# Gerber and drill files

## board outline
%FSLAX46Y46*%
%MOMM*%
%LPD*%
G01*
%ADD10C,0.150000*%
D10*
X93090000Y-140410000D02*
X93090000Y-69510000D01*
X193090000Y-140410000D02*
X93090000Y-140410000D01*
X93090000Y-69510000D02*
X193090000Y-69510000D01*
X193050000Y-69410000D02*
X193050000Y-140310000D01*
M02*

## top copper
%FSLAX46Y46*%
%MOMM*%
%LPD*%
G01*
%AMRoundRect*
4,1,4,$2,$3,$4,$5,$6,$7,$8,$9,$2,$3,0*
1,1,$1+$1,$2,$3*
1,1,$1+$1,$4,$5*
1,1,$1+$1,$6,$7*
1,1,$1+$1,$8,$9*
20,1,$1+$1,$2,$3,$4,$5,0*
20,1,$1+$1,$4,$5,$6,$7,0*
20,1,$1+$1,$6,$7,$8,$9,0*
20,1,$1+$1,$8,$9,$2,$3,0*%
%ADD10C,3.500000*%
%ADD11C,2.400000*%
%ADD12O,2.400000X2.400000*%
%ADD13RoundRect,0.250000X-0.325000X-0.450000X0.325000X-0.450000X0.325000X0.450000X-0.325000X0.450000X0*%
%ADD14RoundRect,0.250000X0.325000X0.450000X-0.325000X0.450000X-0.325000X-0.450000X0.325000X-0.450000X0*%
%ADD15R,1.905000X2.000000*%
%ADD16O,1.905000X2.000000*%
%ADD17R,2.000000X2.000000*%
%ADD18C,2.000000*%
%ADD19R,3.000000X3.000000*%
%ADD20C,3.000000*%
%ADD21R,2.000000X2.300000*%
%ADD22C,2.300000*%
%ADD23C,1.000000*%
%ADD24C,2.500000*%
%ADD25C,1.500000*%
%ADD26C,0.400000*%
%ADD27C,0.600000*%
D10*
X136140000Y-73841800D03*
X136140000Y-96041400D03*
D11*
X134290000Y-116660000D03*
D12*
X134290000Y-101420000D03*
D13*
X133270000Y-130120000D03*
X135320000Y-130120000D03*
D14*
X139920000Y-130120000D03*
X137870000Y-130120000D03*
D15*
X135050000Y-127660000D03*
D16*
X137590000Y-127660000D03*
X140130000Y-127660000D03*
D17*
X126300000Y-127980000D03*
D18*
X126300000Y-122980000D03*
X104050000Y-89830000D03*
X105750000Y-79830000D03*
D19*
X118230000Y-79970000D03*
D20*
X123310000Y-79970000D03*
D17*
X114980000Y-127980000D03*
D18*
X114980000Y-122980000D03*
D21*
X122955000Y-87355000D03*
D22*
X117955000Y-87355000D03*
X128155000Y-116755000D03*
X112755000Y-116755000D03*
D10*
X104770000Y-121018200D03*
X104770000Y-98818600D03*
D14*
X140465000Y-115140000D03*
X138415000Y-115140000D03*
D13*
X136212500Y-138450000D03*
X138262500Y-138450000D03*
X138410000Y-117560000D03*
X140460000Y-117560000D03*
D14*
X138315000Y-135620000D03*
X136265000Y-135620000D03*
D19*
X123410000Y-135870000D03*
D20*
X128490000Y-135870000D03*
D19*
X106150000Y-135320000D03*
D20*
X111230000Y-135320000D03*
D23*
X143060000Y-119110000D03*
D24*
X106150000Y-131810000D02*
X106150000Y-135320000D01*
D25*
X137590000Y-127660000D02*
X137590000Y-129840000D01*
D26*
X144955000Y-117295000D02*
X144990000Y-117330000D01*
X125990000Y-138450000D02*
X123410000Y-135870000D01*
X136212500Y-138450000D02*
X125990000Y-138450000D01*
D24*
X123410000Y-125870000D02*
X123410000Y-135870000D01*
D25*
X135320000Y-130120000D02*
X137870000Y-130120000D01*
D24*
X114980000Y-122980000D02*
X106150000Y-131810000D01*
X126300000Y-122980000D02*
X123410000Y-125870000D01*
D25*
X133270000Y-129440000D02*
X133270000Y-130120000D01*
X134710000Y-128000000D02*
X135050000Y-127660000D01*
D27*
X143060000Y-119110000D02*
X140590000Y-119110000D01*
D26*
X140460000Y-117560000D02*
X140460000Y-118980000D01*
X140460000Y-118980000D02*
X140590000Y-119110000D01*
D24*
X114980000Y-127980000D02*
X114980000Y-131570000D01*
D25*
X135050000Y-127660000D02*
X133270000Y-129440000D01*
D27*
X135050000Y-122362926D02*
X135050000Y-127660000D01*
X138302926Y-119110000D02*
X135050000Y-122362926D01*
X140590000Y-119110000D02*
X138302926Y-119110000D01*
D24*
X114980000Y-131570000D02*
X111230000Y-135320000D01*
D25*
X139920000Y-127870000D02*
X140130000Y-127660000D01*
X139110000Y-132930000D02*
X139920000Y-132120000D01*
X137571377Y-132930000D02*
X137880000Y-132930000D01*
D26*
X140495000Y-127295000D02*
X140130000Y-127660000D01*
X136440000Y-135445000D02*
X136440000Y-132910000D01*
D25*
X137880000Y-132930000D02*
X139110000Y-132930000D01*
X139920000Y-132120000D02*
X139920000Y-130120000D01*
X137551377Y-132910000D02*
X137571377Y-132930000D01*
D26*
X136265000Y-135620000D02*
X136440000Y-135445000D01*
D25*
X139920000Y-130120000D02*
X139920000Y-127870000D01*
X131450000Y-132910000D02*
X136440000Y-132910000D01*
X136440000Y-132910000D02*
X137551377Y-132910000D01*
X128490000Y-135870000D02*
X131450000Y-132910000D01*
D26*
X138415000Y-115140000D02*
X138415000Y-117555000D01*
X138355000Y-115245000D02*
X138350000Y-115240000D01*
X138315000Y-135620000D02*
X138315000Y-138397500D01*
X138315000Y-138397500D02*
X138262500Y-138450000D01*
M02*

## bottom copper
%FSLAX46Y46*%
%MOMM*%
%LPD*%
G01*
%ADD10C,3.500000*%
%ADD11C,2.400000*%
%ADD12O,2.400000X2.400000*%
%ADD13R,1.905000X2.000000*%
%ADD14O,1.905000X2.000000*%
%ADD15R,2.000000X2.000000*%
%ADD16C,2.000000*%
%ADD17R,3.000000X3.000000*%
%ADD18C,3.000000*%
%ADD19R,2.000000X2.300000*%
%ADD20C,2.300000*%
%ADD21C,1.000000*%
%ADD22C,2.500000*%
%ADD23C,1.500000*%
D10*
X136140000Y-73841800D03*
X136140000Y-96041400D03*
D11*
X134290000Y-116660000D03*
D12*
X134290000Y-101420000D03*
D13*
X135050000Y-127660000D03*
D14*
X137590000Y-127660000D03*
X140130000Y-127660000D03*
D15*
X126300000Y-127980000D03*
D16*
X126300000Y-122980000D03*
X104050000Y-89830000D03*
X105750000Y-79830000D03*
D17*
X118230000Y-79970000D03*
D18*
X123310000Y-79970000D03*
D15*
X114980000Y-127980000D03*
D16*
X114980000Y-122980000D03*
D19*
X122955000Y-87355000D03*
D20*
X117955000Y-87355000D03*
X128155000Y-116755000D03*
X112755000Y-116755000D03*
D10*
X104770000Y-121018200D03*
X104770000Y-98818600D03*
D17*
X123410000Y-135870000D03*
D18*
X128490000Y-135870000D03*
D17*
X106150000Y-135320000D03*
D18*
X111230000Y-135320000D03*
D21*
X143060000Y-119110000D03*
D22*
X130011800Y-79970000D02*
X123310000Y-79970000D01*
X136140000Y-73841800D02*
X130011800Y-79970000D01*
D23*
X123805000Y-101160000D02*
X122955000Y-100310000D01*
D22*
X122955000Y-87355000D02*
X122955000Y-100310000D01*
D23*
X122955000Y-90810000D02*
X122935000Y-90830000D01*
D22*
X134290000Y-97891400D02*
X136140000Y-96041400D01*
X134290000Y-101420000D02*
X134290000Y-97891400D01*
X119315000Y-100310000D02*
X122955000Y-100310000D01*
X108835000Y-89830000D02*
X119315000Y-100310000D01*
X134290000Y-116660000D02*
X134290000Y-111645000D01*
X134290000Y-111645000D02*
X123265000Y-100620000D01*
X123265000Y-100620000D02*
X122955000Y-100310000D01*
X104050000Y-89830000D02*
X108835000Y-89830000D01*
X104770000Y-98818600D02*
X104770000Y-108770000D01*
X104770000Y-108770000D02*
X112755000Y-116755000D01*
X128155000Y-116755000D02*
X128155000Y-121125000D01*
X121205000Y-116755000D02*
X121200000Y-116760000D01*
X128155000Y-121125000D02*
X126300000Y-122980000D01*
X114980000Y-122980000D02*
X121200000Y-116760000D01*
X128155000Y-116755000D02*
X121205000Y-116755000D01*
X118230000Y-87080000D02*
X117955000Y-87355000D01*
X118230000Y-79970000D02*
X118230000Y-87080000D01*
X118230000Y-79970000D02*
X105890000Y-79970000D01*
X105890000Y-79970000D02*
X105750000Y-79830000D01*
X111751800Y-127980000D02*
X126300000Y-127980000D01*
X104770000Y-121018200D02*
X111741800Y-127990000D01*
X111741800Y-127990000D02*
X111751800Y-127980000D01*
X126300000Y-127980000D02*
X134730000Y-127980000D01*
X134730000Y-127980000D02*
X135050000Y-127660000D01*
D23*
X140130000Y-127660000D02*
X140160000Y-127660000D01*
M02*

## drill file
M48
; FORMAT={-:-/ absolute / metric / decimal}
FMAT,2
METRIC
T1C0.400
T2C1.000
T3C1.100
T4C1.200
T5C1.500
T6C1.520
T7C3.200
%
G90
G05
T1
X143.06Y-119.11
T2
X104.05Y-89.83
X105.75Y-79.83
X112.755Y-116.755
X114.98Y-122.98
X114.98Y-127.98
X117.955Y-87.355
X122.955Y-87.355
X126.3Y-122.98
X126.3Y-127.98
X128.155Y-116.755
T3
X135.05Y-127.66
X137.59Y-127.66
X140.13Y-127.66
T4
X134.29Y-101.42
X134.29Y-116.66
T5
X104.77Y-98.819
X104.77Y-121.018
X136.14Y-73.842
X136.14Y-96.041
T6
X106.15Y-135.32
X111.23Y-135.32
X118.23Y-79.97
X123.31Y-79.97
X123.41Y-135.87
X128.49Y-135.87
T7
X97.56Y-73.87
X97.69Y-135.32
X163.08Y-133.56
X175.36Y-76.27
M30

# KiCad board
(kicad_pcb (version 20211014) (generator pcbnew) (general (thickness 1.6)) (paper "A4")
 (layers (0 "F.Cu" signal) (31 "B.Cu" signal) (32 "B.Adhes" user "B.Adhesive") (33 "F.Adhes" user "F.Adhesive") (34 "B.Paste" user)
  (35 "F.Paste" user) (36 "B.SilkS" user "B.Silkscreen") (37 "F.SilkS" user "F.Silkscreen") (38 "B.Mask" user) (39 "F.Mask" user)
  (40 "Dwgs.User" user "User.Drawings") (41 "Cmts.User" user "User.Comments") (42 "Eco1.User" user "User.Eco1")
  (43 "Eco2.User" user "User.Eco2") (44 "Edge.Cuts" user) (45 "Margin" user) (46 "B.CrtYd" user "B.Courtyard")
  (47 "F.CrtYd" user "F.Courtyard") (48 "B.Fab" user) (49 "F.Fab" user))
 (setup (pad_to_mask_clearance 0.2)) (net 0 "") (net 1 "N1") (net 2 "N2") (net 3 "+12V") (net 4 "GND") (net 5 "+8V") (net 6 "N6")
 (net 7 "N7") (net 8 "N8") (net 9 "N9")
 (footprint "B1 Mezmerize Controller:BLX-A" (layer "F.Cu") (at 136.14 84.84 -90)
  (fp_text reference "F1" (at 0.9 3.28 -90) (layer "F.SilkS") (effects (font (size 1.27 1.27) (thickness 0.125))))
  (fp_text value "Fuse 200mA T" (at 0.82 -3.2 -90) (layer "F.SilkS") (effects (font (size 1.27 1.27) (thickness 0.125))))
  (pad "1" thru_hole circle locked (at -10.9982 0 270) (size 3.5 3.5) (drill 1.5) (layers *.Cu *.Mask "F.SilkS") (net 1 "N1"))
  (pad "2" thru_hole circle locked (at 11.2014 0 270) (size 3.5 3.5) (drill 1.5) (layers *.Cu *.Mask "F.SilkS") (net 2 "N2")))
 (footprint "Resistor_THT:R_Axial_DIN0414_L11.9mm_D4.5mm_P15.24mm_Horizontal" (layer "F.Cu") (at 134.29 116.66 90)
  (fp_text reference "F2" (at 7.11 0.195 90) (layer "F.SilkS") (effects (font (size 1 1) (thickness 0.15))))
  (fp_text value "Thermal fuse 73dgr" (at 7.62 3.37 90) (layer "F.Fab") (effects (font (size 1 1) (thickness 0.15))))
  (pad "1" thru_hole circle (at 0 0 90) (size 2.4 2.4) (drill 1.2) (layers *.Cu *.Mask) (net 2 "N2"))
  (pad "2" thru_hole oval (at 15.24 0 90) (size 2.4 2.4) (drill 1.2) (layers *.Cu *.Mask) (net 2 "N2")))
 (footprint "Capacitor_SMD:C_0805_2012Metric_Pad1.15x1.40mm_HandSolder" (layer "F.Cu") (at 134.295 130.12)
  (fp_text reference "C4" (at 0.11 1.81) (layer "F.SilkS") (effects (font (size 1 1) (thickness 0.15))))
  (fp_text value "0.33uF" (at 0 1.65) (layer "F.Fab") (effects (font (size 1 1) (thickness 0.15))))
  (pad "1" smd roundrect locked (at -1.025 0) (size 1.15 1.4) (layers "F.Cu" "F.Paste" "F.Mask") (roundrect_rratio 0.217391) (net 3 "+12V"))
  (pad "2" smd roundrect locked (at 1.025 0) (size 1.15 1.4) (layers "F.Cu" "F.Paste" "F.Mask") (roundrect_rratio 0.217391) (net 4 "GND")))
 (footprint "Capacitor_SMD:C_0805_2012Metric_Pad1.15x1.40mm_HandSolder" (layer "F.Cu") (at 138.895 130.12 180)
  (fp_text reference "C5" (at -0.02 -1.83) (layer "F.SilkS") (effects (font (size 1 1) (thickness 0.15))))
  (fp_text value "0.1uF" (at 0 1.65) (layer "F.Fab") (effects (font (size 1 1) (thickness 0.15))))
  (pad "1" smd roundrect locked (at -1.025 0 180) (size 1.15 1.4) (layers "F.Cu" "F.Paste" "F.Mask") (roundrect_rratio 0.217391)
   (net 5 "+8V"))
  (pad "2" smd roundrect locked (at 1.025 0 180) (size 1.15 1.4) (layers "F.Cu" "F.Paste" "F.Mask") (roundrect_rratio 0.217391)
   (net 4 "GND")))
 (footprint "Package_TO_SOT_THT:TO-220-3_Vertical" (layer "F.Cu") (at 135.05 127.66)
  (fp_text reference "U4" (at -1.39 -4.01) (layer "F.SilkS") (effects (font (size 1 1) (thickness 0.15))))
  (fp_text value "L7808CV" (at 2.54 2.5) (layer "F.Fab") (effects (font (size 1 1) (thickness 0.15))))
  (pad "1" thru_hole rect (at 0 0) (size 1.905 2) (drill 1.1) (layers *.Cu *.Mask) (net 3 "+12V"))
  (pad "2" thru_hole oval (at 2.54 0) (size 1.905 2) (drill 1.1) (layers *.Cu *.Mask) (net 4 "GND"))
  (pad "3" thru_hole oval (at 5.08 0) (size 1.905 2) (drill 1.1) (layers *.Cu *.Mask) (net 5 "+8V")))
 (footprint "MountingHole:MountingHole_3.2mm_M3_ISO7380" (layer "F.Cu") (at 163.08 133.56)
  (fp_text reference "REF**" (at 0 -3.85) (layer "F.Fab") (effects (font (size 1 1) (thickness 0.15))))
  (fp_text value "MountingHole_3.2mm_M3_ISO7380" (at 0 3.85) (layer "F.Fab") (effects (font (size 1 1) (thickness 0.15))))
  (pad "" np_thru_hole circle (at 0 0) (size 3.2 3.2) (drill 3.2) (layers *.Cu *.Mask)))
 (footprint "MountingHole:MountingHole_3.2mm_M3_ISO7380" (layer "F.Cu") (at 175.36 76.27)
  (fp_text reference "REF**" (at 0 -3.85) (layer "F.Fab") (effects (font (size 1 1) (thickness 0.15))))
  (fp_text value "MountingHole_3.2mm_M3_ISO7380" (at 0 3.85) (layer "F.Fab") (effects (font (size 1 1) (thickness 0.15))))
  (pad "" np_thru_hole circle (at 0 0) (size 3.2 3.2) (drill 3.2) (layers *.Cu *.Mask)))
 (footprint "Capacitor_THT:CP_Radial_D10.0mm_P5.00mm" (layer "F.Cu") (at 126.3 127.98 90)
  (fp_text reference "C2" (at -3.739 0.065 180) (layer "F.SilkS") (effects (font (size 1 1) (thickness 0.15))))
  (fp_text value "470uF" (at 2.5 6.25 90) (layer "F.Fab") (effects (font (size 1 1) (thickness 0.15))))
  (pad "1" thru_hole rect (at 0 0 90) (size 2 2) (drill 1) (layers *.Cu *.Mask) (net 3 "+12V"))
  (pad "2" thru_hole circle (at 5 0 90) (size 2 2) (drill 1) (layers *.Cu *.Mask) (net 4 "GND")))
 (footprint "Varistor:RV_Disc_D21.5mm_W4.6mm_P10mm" (layer "F.Cu") (at 104.05 89.83 90)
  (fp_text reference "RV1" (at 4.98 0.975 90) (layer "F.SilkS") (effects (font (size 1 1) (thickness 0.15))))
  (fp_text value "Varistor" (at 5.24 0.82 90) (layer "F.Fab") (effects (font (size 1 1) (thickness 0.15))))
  (pad "1" thru_hole circle (at 0 0 90) (size 2 2) (drill 1) (layers *.Cu *.Mask) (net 2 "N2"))
  (pad "2" thru_hole circle (at 10 1.7 90) (size 2 2) (drill 1) (layers *.Cu *.Mask) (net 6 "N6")))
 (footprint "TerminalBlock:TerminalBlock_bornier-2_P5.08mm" (layer "F.Cu") (at 118.23 79.97)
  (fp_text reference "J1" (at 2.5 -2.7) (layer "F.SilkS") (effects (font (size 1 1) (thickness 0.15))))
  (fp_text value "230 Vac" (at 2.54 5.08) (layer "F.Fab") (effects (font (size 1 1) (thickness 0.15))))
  (pad "1" thru_hole rect (at 0 0) (size 3 3) (drill 1.52) (layers *.Cu *.Mask) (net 6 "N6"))
  (pad "2" thru_hole circle (at 5.08 0) (size 3 3) (drill 1.52) (layers *.Cu *.Mask) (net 1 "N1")))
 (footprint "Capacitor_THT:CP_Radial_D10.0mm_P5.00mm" (layer "F.Cu") (at 114.98 127.98 90)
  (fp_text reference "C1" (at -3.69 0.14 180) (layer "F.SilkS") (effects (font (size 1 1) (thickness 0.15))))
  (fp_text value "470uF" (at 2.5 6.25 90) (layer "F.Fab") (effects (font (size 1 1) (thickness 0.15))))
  (pad "1" thru_hole rect (at 0 0 90) (size 2 2) (drill 1) (layers *.Cu *.Mask) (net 3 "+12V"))
  (pad "2" thru_hole circle (at 5 0 90) (size 2 2) (drill 1) (layers *.Cu *.Mask) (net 4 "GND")))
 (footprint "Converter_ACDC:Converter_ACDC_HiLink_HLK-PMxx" (layer "F.Cu") (at 122.955 87.355 -90)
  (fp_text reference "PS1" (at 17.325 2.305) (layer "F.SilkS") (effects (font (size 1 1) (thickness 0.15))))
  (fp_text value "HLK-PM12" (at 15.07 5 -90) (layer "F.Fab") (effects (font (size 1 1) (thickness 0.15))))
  (pad "1" thru_hole rect (at 0 0 270) (size 2.3 2) (drill 1) (layers *.Cu *.Mask) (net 2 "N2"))
  (pad "2" thru_hole circle (at 0 5 270) (size 2.3 2.3) (drill 1) (layers *.Cu *.Mask) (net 6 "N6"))
  (pad "3" thru_hole circle (at 29.4 -5.2 270) (size 2.3 2.3) (drill 1) (layers *.Cu *.Mask) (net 4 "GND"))
  (pad "4" thru_hole circle (at 29.4 10.2 270) (size 2.3 2.3) (drill 1) (layers *.Cu *.Mask) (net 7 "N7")))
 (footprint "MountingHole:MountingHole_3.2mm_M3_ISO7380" (layer "F.Cu") (at 97.56 73.87)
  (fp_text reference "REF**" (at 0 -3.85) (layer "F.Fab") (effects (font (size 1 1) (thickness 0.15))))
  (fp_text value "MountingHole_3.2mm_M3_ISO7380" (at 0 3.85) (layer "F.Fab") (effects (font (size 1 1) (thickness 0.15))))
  (pad "" np_thru_hole circle (at 0 0) (size 3.2 3.2) (drill 3.2) (layers *.Cu *.Mask)))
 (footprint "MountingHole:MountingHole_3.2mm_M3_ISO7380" (layer "F.Cu") (at 97.69 135.32)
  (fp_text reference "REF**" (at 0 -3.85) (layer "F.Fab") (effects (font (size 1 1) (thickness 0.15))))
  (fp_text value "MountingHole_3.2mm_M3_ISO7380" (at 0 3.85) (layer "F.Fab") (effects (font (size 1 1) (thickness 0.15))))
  (pad "" np_thru_hole circle (at 0 0) (size 3.2 3.2) (drill 3.2) (layers *.Cu *.Mask)))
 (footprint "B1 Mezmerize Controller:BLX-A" (layer "F.Cu") (at 104.77 110.02 90)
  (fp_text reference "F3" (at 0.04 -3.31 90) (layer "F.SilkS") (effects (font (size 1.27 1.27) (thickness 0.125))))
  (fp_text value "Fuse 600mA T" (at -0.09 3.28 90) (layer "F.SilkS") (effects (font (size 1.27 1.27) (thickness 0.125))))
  (pad "1" thru_hole circle locked (at -10.9982 0 90) (size 3.5 3.5) (drill 1.5) (layers *.Cu *.Mask "F.SilkS") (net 3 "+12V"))
  (pad "2" thru_hole circle locked (at 11.2014 0 90) (size 3.5 3.5) (drill 1.5) (layers *.Cu *.Mask "F.SilkS") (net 7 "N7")))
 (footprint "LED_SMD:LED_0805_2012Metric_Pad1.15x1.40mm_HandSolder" (layer "F.Cu") (at 139.44 115.14 180)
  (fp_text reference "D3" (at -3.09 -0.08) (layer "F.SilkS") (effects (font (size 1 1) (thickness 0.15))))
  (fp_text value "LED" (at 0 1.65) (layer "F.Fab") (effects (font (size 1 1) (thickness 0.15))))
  (pad "1" smd roundrect (at -1.025 0 180) (size 1.15 1.4) (layers "F.Cu" "F.Paste" "F.Mask") (roundrect_rratio 0.217391) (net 4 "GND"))
  (pad "2" smd roundrect (at 1.025 0 180) (size 1.15 1.4) (layers "F.Cu" "F.Paste" "F.Mask") (roundrect_rratio 0.217391) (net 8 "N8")))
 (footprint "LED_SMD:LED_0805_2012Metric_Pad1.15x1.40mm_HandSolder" (layer "F.Cu") (at 137.2375 138.45)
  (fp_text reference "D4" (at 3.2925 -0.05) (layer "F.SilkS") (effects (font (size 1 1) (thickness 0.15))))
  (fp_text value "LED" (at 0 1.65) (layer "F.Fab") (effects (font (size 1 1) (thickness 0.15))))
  (pad "1" smd roundrect (at -1.025 0) (size 1.15 1.4) (layers "F.Cu" "F.Paste" "F.Mask") (roundrect_rratio 0.217391) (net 4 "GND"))
  (pad "2" smd roundrect (at 1.025 0) (size 1.15 1.4) (layers "F.Cu" "F.Paste" "F.Mask") (roundrect_rratio 0.217391) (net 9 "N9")))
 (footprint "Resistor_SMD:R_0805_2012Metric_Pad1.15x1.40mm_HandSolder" (layer "F.Cu") (at 139.435 117.56)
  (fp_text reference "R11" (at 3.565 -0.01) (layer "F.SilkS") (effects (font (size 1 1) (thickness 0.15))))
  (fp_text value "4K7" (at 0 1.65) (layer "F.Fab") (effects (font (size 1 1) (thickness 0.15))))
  (pad "1" smd roundrect locked (at -1.025 0) (size 1.15 1.4) (layers "F.Cu" "F.Paste" "F.Mask") (roundrect_rratio 0.217391) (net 8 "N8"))
  (pad "2" smd roundrect locked (at 1.025 0) (size 1.15 1.4) (layers "F.Cu" "F.Paste" "F.Mask") (roundrect_rratio 0.217391) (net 3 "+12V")))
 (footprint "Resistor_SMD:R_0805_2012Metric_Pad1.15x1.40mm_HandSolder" (layer "F.Cu") (at 137.29 135.62 180)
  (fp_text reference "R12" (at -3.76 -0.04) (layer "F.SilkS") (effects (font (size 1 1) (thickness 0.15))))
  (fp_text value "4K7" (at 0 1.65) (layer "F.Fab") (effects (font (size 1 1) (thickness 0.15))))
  (pad "1" smd roundrect locked (at -1.025 0 180) (size 1.15 1.4) (layers "F.Cu" "F.Paste" "F.Mask") (roundrect_rratio 0.217391)
   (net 9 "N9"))
  (pad "2" smd roundrect locked (at 1.025 0 180) (size 1.15 1.4) (layers "F.Cu" "F.Paste" "F.Mask") (roundrect_rratio 0.217391)
   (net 5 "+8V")))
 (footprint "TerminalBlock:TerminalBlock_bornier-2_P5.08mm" (layer "F.Cu") (at 123.41 135.87)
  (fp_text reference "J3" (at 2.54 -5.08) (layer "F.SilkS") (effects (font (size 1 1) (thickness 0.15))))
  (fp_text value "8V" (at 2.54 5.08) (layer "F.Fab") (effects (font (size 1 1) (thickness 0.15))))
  (pad "1" thru_hole rect (at 0 0) (size 3 3) (drill 1.52) (layers *.Cu *.Mask) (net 4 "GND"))
  (pad "2" thru_hole circle (at 5.08 0) (size 3 3) (drill 1.52) (layers *.Cu *.Mask) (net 5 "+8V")))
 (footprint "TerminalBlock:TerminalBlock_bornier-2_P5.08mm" (layer "F.Cu") (at 106.15 135.32)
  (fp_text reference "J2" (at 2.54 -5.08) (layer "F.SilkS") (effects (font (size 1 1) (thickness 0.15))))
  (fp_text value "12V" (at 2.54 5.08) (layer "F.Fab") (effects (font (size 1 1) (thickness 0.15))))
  (pad "1" thru_hole rect (at 0 0) (size 3 3) (drill 1.52) (layers *.Cu *.Mask) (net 4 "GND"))
  (pad "2" thru_hole circle (at 5.08 0) (size 3 3) (drill 1.52) (layers *.Cu *.Mask) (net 3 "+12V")))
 (gr_line (start 93.09 140.41) (end 93.09 69.51) (layer "Edge.Cuts") (width 0.15))
 (gr_line (start 193.09 140.41) (end 93.09 140.41) (layer "Edge.Cuts") (width 0.15))
 (gr_line (start 93.09 69.51) (end 193.09 69.51) (layer "Edge.Cuts") (width 0.15))
 (gr_line (start 193.05 69.41) (end 193.05 140.31) (layer "Edge.Cuts") (width 0.15))
 (segment (start 130.0118 79.97) (end 123.31 79.97) (width 2.5) (layer "B.Cu") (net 1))
 (segment (start 136.14 73.8418) (end 130.0118 79.97) (width 2.5) (layer "B.Cu") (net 1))
 (segment (start 123.805 101.16) (end 122.955 100.31) (width 1.5) (layer "B.Cu") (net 2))
 (segment (start 122.955 87.355) (end 122.955 100.31) (width 2.5) (layer "B.Cu") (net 2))
 (segment (start 122.955 90.81) (end 122.935 90.83) (width 1.5) (layer "B.Cu") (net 2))
 (segment (start 134.29 97.8914) (end 136.14 96.0414) (width 2.5) (layer "B.Cu") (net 2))
 (segment (start 134.29 101.42) (end 134.29 97.8914) (width 2.5) (layer "B.Cu") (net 2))
 (segment (start 119.315 100.31) (end 122.955 100.31) (width 2.5) (layer "B.Cu") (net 2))
 (segment (start 108.835 89.83) (end 119.315 100.31) (width 2.5) (layer "B.Cu") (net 2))
 (segment (start 134.29 116.66) (end 134.29 111.645) (width 2.5) (layer "B.Cu") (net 2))
 (segment (start 134.29 111.645) (end 123.265 100.62) (width 2.5) (layer "B.Cu") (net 2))
 (segment (start 123.265 100.62) (end 122.955 100.31) (width 2.5) (layer "B.Cu") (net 2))
 (segment (start 104.05 89.83) (end 108.835 89.83) (width 2.5) (layer "B.Cu") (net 2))
 (segment (start 104.77 98.8186) (end 104.77 108.77) (width 2.5) (layer "B.Cu") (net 7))
 (segment (start 104.77 108.77) (end 112.755 116.755) (width 2.5) (layer "B.Cu") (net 7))
 (segment (start 106.15 131.81) (end 106.15 135.32) (width 2.5) (layer "F.Cu") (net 4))
 (segment (start 137.59 127.66) (end 137.59 129.84) (width 1.5) (layer "F.Cu") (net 4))
 (segment (start 144.955 117.295) (end 144.99 117.33) (width 0.4) (layer "F.Cu") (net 4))
 (segment (start 125.99 138.45) (end 123.41 135.87) (width 0.4) (layer "F.Cu") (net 4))
 (segment (start 136.2125 138.45) (end 125.99 138.45) (width 0.4) (layer "F.Cu") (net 4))
 (segment (start 123.41 125.87) (end 123.41 135.87) (width 2.5) (layer "F.Cu") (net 4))
 (segment (start 135.32 130.12) (end 137.87 130.12) (width 1.5) (layer "F.Cu") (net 4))
 (segment (start 114.98 122.98) (end 106.15 131.81) (width 2.5) (layer "F.Cu") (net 4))
 (segment (start 126.3 122.98) (end 123.41 125.87) (width 2.5) (layer "F.Cu") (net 4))
 (segment (start 128.155 116.755) (end 128.155 121.125) (width 2.5) (layer "B.Cu") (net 4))
 (segment (start 121.205 116.755) (end 121.2 116.76) (width 2.5) (layer "B.Cu") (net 4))
 (segment (start 128.155 121.125) (end 126.3 122.98) (width 2.5) (layer "B.Cu") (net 4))
 (segment (start 114.98 122.98) (end 121.2 116.76) (width 2.5) (layer "B.Cu") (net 4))
 (segment (start 128.155 116.755) (end 121.205 116.755) (width 2.5) (layer "B.Cu") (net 4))
 (segment (start 118.23 87.08) (end 117.955 87.355) (width 2.5) (layer "B.Cu") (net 6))
 (segment (start 118.23 79.97) (end 118.23 87.08) (width 2.5) (layer "B.Cu") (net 6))
 (segment (start 118.23 79.97) (end 105.89 79.97) (width 2.5) (layer "B.Cu") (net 6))
 (segment (start 105.89 79.97) (end 105.75 79.83) (width 2.5) (layer "B.Cu") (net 6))
 (segment (start 133.27 129.44) (end 133.27 130.12) (width 1.5) (layer "F.Cu") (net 3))
 (segment (start 134.71 128) (end 135.05 127.66) (width 1.5) (layer "F.Cu") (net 3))
 (segment (start 143.06 119.11) (end 140.59 119.11) (width 0.6) (layer "F.Cu") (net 3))
 (segment (start 140.46 117.56) (end 140.46 118.98) (width 0.4) (layer "F.Cu") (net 3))
 (segment (start 140.46 118.98) (end 140.59 119.11) (width 0.4) (layer "F.Cu") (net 3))
 (segment (start 114.98 127.98) (end 114.98 131.57) (width 2.5) (layer "F.Cu") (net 3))
 (segment (start 135.05 127.66) (end 133.27 129.44) (width 1.5) (layer "F.Cu") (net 3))
 (segment (start 135.05 122.362926) (end 135.05 127.66) (width 0.6) (layer "F.Cu") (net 3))
 (segment (start 138.302926 119.11) (end 135.05 122.362926) (width 0.6) (layer "F.Cu") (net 3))
 (segment (start 140.59 119.11) (end 138.302926 119.11) (width 0.6) (layer "F.Cu") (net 3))
 (segment (start 114.98 131.57) (end 111.23 135.32) (width 2.5) (layer "F.Cu") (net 3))
 (via (at 143.06 119.11) (size 1) (drill 0.4) (layers "F.Cu" "B.Cu") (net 3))
 (segment (start 111.7518 127.98) (end 126.3 127.98) (width 2.5) (layer "B.Cu") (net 3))
 (segment (start 104.77 121.0182) (end 111.7418 127.99) (width 2.5) (layer "B.Cu") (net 3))
 (segment (start 111.7418 127.99) (end 111.7518 127.98) (width 2.5) (layer "B.Cu") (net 3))
 (segment (start 126.3 127.98) (end 134.73 127.98) (width 2.5) (layer "B.Cu") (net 3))
 (segment (start 134.73 127.98) (end 135.05 127.66) (width 2.5) (layer "B.Cu") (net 3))
 (segment (start 139.92 127.87) (end 140.13 127.66) (width 1.5) (layer "F.Cu") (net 5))
 (segment (start 139.11 132.93) (end 139.92 132.12) (width 1.5) (layer "F.Cu") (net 5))
 (segment (start 137.571377 132.93) (end 137.88 132.93) (width 1.5) (layer "F.Cu") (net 5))
 (segment (start 140.495 127.295) (end 140.13 127.66) (width 0.4) (layer "F.Cu") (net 5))
 (segment (start 136.44 135.445) (end 136.44 132.91) (width 0.4) (layer "F.Cu") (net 5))
 (segment (start 137.88 132.93) (end 139.11 132.93) (width 1.5) (layer "F.Cu") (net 5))
 (segment (start 139.92 132.12) (end 139.92 130.12) (width 1.5) (layer "F.Cu") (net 5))
 (segment (start 137.551377 132.91) (end 137.571377 132.93) (width 1.5) (layer "F.Cu") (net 5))
 (segment (start 136.265 135.62) (end 136.44 135.445) (width 0.4) (layer "F.Cu") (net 5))
 (segment (start 139.92 130.12) (end 139.92 127.87) (width 1.5) (layer "F.Cu") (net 5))
 (segment (start 131.45 132.91) (end 136.44 132.91) (width 1.5) (layer "F.Cu") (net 5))
 (segment (start 136.44 132.91) (end 137.551377 132.91) (width 1.5) (layer "F.Cu") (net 5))
 (segment (start 128.49 135.87) (end 131.45 132.91) (width 1.5) (layer "F.Cu") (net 5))
 (segment (start 140.13 127.66) (end 140.16 127.66) (width 1.5) (layer "B.Cu") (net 5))
 (segment (start 138.415 115.14) (end 138.415 117.555) (width 0.4) (layer "F.Cu") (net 8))
 (segment (start 138.355 115.245) (end 138.35 115.24) (width 0.4) (layer "F.Cu") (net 8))
 (segment (start 138.315 135.62) (end 138.315 138.3975) (width 0.4) (layer "F.Cu") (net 9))
 (segment (start 138.315 138.3975) (end 138.2625 138.45) (width 0.4) (layer "F.Cu") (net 9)))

